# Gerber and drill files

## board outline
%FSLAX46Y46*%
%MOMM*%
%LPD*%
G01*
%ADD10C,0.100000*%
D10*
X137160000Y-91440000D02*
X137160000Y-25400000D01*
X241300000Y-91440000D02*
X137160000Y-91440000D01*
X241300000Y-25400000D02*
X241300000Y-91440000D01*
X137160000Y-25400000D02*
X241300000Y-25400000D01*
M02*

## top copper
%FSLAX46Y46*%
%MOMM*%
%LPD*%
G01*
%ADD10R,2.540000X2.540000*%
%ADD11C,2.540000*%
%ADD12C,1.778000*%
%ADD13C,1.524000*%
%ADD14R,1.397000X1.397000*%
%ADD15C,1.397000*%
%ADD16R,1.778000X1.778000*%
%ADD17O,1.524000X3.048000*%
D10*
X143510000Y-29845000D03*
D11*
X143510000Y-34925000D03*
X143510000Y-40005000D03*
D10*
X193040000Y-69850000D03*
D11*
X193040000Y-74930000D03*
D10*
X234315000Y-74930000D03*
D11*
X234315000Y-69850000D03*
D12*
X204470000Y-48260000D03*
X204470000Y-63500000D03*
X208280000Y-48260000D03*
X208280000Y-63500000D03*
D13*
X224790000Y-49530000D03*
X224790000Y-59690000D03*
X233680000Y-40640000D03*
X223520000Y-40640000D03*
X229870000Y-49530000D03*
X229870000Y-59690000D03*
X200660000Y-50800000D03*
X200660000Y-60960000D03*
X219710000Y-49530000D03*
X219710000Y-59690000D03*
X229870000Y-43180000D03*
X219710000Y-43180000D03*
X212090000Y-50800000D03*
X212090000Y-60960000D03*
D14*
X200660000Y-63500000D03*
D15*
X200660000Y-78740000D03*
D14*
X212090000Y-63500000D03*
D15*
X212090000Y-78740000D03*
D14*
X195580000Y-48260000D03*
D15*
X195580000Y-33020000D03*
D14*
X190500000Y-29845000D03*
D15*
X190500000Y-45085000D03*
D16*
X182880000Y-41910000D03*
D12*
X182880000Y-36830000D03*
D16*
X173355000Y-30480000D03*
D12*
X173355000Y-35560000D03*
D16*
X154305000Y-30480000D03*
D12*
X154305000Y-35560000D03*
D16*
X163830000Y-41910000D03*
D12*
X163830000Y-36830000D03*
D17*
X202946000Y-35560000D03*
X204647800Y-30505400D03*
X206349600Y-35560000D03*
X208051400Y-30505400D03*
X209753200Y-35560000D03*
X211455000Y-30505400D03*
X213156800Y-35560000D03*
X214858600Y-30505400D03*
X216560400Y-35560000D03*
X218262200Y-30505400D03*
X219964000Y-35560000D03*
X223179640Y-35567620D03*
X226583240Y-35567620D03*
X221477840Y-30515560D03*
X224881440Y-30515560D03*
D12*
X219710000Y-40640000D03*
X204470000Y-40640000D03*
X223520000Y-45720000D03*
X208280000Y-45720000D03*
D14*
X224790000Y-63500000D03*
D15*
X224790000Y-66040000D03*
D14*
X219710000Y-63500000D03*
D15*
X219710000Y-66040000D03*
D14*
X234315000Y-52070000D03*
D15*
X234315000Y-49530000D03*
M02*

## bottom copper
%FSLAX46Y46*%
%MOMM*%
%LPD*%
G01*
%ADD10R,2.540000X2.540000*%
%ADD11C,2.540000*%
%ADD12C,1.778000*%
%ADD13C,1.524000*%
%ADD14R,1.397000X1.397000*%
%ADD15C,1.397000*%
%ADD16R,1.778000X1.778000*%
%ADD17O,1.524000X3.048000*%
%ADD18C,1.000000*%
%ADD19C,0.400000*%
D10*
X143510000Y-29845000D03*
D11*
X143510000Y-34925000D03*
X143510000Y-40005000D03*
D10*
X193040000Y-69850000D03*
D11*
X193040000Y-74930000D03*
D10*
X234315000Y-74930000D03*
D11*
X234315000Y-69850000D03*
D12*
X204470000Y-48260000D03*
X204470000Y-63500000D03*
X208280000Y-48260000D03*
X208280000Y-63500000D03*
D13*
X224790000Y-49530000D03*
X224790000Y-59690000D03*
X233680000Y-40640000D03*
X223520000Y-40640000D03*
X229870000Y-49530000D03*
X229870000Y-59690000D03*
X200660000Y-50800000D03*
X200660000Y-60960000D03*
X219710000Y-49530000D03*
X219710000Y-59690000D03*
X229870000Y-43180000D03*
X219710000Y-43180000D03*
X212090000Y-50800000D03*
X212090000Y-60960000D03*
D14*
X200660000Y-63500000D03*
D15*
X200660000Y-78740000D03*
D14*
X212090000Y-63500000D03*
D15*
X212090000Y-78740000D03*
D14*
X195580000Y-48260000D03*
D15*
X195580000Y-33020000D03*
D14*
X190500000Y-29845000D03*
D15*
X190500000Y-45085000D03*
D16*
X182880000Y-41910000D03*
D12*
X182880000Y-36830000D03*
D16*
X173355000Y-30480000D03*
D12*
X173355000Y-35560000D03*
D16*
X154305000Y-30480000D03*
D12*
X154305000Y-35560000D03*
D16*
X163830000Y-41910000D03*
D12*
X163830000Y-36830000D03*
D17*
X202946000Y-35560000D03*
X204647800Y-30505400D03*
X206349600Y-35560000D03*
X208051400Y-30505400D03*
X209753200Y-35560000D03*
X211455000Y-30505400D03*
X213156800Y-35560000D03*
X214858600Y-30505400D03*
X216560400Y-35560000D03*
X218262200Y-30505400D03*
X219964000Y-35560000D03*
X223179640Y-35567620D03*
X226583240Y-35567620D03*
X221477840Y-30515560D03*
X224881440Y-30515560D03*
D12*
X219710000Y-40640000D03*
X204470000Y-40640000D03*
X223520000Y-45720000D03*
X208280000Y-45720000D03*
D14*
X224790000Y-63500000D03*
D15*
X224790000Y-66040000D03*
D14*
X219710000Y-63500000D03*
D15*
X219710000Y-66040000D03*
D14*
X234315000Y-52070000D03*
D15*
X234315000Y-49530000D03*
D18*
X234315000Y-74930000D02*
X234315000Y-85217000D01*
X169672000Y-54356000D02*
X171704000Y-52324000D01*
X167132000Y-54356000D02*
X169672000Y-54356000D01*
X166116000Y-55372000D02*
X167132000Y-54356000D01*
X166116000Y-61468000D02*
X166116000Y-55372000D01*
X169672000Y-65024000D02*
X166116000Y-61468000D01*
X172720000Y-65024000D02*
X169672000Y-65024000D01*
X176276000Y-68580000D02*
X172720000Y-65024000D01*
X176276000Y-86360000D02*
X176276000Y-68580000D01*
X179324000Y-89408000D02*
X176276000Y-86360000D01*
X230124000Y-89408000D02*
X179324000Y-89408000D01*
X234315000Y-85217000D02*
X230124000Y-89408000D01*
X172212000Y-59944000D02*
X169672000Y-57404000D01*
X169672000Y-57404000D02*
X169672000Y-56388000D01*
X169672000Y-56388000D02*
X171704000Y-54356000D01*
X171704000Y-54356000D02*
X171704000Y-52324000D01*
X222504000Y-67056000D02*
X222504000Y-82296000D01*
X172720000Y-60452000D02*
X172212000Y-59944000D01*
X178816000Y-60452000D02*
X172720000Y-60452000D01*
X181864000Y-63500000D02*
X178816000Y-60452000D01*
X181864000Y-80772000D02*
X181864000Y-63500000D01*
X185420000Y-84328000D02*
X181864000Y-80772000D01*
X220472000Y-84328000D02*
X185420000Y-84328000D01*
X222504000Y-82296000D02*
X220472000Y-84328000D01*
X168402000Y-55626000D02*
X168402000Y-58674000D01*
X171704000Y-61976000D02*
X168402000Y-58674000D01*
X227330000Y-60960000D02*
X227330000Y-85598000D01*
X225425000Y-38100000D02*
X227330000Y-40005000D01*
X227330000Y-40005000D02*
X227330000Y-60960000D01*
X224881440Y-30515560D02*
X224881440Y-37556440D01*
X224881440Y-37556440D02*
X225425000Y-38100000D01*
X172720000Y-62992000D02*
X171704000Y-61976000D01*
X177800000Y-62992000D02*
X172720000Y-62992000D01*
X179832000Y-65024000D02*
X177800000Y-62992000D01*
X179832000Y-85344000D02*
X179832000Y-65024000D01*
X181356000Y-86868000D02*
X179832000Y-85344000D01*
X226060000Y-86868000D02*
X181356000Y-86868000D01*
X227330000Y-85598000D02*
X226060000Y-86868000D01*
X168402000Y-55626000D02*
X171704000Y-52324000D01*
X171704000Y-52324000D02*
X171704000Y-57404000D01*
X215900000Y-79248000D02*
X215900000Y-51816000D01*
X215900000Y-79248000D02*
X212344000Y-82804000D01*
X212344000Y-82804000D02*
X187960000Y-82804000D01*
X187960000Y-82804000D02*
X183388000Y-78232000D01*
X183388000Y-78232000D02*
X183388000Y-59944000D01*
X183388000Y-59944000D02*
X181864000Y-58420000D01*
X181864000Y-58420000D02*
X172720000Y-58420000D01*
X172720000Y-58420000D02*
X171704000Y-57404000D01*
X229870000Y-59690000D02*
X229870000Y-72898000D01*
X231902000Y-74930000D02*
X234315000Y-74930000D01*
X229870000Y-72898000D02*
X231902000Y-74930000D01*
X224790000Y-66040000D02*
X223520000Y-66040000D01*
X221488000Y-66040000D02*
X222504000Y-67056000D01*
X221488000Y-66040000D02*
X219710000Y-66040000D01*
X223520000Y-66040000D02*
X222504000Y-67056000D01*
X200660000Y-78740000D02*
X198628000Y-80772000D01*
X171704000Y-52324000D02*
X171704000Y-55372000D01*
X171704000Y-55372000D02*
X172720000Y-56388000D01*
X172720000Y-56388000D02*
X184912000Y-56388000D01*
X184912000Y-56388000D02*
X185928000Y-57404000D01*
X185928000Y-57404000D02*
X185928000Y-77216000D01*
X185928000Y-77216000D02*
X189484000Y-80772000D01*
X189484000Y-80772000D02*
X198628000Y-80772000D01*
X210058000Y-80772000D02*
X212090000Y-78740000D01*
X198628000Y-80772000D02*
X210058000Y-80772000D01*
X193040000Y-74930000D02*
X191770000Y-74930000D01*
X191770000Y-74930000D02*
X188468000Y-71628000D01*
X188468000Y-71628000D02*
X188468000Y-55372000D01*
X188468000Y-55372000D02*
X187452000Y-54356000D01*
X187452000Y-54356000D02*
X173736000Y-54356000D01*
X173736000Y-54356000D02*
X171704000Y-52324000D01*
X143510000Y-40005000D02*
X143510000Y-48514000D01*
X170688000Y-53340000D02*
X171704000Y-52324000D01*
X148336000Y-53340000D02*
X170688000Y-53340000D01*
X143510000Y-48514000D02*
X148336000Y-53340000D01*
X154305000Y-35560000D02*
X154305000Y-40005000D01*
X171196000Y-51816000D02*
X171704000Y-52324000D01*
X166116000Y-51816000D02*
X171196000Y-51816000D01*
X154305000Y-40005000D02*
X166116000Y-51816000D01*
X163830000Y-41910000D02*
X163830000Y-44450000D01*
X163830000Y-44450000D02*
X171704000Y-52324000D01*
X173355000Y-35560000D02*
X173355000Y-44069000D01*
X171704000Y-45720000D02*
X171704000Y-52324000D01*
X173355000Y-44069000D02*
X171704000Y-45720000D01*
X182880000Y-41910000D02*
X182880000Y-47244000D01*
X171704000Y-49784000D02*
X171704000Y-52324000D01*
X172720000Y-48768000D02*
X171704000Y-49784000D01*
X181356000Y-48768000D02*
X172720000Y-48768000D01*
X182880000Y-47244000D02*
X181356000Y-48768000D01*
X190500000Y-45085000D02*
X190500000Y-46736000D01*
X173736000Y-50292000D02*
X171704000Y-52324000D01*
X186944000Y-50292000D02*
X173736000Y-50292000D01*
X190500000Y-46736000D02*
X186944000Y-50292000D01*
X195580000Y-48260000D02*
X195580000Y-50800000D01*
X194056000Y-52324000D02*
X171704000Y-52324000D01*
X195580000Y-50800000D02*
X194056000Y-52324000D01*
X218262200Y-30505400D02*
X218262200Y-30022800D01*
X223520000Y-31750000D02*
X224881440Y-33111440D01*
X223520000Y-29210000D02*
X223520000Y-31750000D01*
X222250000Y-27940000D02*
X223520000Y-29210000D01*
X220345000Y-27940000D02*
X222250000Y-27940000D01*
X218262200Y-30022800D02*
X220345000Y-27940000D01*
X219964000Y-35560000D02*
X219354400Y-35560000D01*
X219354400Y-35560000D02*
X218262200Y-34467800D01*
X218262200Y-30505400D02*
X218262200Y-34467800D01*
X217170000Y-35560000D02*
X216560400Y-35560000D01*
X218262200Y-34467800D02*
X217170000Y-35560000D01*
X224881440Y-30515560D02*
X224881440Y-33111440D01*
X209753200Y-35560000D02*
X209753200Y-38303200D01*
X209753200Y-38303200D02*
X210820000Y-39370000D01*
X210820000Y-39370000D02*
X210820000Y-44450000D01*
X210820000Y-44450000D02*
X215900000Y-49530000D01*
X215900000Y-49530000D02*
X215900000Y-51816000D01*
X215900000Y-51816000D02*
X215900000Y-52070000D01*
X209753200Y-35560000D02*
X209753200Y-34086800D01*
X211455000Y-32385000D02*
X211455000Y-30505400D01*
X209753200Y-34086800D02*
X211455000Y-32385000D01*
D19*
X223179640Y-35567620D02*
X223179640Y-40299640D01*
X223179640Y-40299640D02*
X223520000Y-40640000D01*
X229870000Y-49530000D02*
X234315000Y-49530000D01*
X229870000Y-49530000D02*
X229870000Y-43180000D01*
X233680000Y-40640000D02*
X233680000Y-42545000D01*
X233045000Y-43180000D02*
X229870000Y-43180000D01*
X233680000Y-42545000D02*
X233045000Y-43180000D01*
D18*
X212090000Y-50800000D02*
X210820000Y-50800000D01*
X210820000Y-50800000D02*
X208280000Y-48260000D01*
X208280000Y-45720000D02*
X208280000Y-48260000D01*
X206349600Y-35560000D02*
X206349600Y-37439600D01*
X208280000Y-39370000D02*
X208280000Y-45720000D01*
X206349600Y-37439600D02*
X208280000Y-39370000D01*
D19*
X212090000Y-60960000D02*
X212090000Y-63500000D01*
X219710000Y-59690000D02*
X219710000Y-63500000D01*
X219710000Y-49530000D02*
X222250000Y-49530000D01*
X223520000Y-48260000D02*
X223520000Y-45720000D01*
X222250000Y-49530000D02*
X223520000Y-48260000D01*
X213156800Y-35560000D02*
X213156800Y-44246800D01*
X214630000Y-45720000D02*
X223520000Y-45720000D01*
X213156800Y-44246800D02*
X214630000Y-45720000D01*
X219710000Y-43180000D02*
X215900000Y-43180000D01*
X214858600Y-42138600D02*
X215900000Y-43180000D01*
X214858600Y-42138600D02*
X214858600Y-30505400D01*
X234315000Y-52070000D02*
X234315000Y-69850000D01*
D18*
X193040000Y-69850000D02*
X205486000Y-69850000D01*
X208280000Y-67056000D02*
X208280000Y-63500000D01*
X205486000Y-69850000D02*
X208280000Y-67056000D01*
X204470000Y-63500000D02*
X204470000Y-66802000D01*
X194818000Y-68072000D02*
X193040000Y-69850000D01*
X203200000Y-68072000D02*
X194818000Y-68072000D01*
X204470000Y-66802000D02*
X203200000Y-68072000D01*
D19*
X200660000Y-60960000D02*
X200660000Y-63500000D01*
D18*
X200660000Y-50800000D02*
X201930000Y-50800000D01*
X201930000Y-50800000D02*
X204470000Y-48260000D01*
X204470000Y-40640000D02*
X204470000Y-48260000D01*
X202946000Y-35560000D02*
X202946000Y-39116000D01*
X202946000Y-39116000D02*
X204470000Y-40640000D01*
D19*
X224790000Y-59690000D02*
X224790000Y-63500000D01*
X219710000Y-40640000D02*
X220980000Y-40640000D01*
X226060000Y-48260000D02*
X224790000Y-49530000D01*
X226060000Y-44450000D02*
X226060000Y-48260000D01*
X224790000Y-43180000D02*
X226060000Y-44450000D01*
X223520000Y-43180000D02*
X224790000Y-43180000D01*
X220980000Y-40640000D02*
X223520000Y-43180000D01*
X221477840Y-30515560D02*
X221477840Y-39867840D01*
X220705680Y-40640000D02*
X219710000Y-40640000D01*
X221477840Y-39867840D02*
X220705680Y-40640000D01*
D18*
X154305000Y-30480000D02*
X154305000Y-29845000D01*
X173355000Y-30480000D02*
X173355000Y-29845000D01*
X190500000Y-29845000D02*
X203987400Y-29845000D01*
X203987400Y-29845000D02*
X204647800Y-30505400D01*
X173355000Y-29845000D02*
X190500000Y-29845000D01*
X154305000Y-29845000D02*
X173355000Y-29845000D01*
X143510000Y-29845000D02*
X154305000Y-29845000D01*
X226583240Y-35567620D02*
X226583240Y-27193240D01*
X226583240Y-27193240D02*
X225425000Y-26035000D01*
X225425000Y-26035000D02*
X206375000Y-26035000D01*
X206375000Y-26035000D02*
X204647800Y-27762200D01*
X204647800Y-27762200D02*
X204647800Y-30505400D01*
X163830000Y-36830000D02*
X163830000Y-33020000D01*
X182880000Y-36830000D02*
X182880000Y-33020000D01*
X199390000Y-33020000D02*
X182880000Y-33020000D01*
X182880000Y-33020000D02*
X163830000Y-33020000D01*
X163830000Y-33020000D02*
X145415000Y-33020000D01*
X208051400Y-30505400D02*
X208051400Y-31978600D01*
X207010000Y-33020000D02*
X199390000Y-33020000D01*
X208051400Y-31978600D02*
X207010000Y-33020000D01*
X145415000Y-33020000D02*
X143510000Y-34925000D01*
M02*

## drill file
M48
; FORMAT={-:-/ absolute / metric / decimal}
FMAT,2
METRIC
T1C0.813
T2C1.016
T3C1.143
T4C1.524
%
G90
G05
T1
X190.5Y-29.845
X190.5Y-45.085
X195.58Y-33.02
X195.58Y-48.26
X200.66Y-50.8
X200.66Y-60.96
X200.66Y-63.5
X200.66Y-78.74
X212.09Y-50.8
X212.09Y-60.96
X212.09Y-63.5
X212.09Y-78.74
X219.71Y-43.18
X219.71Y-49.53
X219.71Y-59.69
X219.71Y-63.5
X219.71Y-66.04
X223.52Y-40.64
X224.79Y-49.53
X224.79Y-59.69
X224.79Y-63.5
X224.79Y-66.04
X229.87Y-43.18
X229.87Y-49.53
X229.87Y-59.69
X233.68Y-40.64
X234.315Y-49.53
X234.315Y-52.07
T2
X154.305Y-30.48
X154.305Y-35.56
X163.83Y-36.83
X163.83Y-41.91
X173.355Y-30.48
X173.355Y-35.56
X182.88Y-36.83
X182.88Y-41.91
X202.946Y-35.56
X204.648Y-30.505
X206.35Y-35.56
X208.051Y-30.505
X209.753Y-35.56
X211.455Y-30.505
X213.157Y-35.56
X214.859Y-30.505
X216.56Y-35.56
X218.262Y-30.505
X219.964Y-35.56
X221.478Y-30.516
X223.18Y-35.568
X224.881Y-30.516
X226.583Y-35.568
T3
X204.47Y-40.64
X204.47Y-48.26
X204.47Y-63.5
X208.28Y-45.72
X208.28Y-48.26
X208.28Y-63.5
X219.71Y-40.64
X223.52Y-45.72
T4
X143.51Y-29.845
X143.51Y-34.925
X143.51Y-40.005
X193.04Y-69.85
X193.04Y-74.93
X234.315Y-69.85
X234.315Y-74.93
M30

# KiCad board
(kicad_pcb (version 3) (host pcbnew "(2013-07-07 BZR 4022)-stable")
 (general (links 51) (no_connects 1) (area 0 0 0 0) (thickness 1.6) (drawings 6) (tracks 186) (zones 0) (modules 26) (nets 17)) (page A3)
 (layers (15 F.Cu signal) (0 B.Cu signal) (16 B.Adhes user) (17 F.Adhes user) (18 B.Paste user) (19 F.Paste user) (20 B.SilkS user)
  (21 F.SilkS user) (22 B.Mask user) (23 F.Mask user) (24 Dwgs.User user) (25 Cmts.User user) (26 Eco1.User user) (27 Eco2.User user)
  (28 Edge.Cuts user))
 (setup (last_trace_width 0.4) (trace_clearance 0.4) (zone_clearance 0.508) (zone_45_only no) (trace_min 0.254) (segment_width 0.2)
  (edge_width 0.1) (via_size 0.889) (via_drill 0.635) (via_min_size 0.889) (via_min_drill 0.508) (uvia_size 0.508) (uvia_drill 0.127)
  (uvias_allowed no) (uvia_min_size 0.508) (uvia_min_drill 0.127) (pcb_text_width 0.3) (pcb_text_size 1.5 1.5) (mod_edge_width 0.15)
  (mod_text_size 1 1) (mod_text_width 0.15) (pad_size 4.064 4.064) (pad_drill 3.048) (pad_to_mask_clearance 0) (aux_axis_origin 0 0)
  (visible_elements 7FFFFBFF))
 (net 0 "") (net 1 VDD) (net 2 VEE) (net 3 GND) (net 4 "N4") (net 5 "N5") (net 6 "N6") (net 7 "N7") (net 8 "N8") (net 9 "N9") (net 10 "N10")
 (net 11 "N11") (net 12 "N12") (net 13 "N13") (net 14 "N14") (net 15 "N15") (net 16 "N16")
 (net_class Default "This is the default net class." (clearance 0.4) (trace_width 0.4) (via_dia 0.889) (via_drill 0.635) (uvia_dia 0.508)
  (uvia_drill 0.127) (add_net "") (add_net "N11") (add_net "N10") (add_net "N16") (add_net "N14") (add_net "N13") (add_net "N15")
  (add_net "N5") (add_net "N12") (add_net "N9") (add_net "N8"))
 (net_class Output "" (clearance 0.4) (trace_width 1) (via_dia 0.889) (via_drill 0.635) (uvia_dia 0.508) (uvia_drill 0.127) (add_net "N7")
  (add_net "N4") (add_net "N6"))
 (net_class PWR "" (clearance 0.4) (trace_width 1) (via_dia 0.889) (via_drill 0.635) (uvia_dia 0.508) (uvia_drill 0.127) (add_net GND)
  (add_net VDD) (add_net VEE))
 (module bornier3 (layer F.Cu) (at 143.51 34.925 270)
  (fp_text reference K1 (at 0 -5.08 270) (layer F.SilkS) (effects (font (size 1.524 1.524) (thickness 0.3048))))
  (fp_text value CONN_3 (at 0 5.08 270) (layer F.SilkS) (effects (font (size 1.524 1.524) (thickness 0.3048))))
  (pad 1 thru_hole rect (at -5.08 0 270) (size 2.54 2.54) (drill 1.524) (layers *.Cu *.Mask F.SilkS) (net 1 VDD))
  (pad 2 thru_hole circle (at 0 0 270) (size 2.54 2.54) (drill 1.524) (layers *.Cu *.Mask F.SilkS) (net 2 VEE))
  (pad 3 thru_hole circle (at 5.08 0 270) (size 2.54 2.54) (drill 1.524) (layers *.Cu *.Mask F.SilkS) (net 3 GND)))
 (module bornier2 (layer F.Cu) (at 193.04 72.39 270)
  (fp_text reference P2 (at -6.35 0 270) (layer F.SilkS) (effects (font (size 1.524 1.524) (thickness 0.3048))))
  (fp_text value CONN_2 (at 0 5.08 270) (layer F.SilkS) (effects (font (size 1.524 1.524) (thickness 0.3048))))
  (pad 1 thru_hole rect (at -2.54 0 270) (size 2.54 2.54) (drill 1.524) (layers *.Cu *.Mask F.SilkS) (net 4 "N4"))
  (pad 2 thru_hole circle (at 2.54 0 270) (size 2.54 2.54) (drill 1.524) (layers *.Cu *.Mask F.SilkS) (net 3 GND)))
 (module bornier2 (layer F.Cu) (at 234.315 72.39 90)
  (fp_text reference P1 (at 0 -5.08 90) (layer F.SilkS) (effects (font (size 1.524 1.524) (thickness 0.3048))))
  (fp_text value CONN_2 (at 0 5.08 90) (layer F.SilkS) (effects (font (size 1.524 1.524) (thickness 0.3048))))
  (pad 1 thru_hole rect (at -2.54 0 90) (size 2.54 2.54) (drill 1.524) (layers *.Cu *.Mask F.SilkS) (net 3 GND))
  (pad 2 thru_hole circle (at 2.54 0 90) (size 2.54 2.54) (drill 1.524) (layers *.Cu *.Mask F.SilkS) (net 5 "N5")))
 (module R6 (layer F.Cu) (at 204.47 55.88 270) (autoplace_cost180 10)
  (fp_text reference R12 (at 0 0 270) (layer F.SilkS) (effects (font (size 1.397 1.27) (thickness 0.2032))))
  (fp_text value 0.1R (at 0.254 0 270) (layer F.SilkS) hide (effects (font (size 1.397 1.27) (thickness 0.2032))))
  (pad 1 thru_hole circle (at -7.62 0 270) (size 1.778 1.778) (drill 1.143) (layers *.Cu *.Mask F.SilkS) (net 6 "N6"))
  (pad 2 thru_hole circle (at 7.62 0 270) (size 1.778 1.778) (drill 1.143) (layers *.Cu *.Mask F.SilkS) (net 4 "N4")))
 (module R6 (layer F.Cu) (at 208.28 55.88 270) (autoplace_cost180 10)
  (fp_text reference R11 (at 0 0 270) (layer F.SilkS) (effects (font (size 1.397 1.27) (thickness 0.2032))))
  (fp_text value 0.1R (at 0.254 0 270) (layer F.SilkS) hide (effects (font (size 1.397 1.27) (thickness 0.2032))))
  (pad 1 thru_hole circle (at -7.62 0 270) (size 1.778 1.778) (drill 1.143) (layers *.Cu *.Mask F.SilkS) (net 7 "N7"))
  (pad 2 thru_hole circle (at 7.62 0 270) (size 1.778 1.778) (drill 1.143) (layers *.Cu *.Mask F.SilkS) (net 4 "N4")))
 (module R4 (layer F.Cu) (at 224.79 54.61 270) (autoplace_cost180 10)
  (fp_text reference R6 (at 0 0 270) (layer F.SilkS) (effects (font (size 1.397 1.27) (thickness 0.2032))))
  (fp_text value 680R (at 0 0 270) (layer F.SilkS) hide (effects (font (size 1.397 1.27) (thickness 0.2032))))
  (pad 1 thru_hole circle (at -5.08 0 270) (size 1.524 1.524) (drill 0.8128) (layers *.Cu *.Mask F.SilkS) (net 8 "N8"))
  (pad 2 thru_hole circle (at 5.08 0 270) (size 1.524 1.524) (drill 0.8128) (layers *.Cu *.Mask F.SilkS) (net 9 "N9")))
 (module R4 (layer F.Cu) (at 228.6 40.64 180) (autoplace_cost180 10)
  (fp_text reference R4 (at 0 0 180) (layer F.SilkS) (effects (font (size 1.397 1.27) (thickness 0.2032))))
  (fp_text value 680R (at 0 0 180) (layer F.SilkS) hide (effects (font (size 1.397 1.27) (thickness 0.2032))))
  (pad 1 thru_hole circle (at -5.08 0 180) (size 1.524 1.524) (drill 0.8128) (layers *.Cu *.Mask F.SilkS) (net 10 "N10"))
  (pad 2 thru_hole circle (at 5.08 0 180) (size 1.524 1.524) (drill 0.8128) (layers *.Cu *.Mask F.SilkS) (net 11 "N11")))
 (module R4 (layer F.Cu) (at 229.87 54.61 270) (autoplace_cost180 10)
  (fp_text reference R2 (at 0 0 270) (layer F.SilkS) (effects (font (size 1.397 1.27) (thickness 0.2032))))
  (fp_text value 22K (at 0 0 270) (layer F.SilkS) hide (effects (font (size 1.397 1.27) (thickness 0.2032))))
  (pad 1 thru_hole circle (at -5.08 0 270) (size 1.524 1.524) (drill 0.8128) (layers *.Cu *.Mask F.SilkS) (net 10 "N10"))
  (pad 2 thru_hole circle (at 5.08 0 270) (size 1.524 1.524) (drill 0.8128) (layers *.Cu *.Mask F.SilkS) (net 3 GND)))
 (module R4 (layer F.Cu) (at 200.66 55.88 270) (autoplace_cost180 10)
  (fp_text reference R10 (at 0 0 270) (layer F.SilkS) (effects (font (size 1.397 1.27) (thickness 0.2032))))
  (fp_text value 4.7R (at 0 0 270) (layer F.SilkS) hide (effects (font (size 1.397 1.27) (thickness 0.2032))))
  (pad 1 thru_hole circle (at -5.08 0 270) (size 1.524 1.524) (drill 0.8128) (layers *.Cu *.Mask F.SilkS) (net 6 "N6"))
  (pad 2 thru_hole circle (at 5.08 0 270) (size 1.524 1.524) (drill 0.8128) (layers *.Cu *.Mask F.SilkS) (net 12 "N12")))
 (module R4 (layer F.Cu) (at 219.71 54.61 270) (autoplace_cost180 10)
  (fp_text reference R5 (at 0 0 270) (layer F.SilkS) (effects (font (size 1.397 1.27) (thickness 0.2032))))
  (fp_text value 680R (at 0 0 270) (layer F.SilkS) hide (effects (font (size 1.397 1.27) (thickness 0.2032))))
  (pad 1 thru_hole circle (at -5.08 0 270) (size 1.524 1.524) (drill 0.8128) (layers *.Cu *.Mask F.SilkS) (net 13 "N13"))
  (pad 2 thru_hole circle (at 5.08 0 270) (size 1.524 1.524) (drill 0.8128) (layers *.Cu *.Mask F.SilkS) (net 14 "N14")))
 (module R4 (layer F.Cu) (at 224.79 43.18 180) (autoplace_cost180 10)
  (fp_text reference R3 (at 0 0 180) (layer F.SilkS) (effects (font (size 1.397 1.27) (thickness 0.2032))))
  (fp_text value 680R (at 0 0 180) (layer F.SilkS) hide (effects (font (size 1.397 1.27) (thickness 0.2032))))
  (pad 1 thru_hole circle (at -5.08 0 180) (size 1.524 1.524) (drill 0.8128) (layers *.Cu *.Mask F.SilkS) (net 10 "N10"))
  (pad 2 thru_hole circle (at 5.08 0 180) (size 1.524 1.524) (drill 0.8128) (layers *.Cu *.Mask F.SilkS) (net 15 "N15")))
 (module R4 (layer F.Cu) (at 212.09 55.88 270) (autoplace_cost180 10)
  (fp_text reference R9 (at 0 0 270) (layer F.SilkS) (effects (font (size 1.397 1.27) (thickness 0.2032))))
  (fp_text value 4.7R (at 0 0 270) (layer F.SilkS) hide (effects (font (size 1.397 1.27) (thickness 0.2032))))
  (pad 1 thru_hole circle (at -5.08 0 270) (size 1.524 1.524) (drill 0.8128) (layers *.Cu *.Mask F.SilkS) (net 7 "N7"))
  (pad 2 thru_hole circle (at 5.08 0 270) (size 1.524 1.524) (drill 0.8128) (layers *.Cu *.Mask F.SilkS) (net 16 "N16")))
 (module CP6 (layer F.Cu) (at 200.66 71.12 270)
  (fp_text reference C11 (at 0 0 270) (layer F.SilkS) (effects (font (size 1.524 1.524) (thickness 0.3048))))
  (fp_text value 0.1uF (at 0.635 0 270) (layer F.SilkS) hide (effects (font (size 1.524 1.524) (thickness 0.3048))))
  (pad 1 thru_hole rect (at -7.62 0 270) (size 1.397 1.397) (drill 0.8128) (layers *.Cu *.Mask F.SilkS) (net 12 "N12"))
  (pad 2 thru_hole circle (at 7.62 0 270) (size 1.397 1.397) (drill 0.8128) (layers *.Cu *.Mask F.SilkS) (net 3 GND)))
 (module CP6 (layer F.Cu) (at 212.09 71.12 270)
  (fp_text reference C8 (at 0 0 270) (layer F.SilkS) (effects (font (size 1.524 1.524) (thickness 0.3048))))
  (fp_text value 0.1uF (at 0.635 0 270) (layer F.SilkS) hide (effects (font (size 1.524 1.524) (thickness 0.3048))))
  (pad 1 thru_hole rect (at -7.62 0 270) (size 1.397 1.397) (drill 0.8128) (layers *.Cu *.Mask F.SilkS) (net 16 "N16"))
  (pad 2 thru_hole circle (at 7.62 0 270) (size 1.397 1.397) (drill 0.8128) (layers *.Cu *.Mask F.SilkS) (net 3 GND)))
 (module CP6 (layer F.Cu) (at 195.58 40.64 90)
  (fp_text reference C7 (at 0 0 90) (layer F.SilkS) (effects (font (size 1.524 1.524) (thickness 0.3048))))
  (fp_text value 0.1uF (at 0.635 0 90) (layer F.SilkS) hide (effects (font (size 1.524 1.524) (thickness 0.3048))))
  (pad 1 thru_hole rect (at -7.62 0 90) (size 1.397 1.397) (drill 0.8128) (layers *.Cu *.Mask F.SilkS) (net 3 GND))
  (pad 2 thru_hole circle (at 7.62 0 90) (size 1.397 1.397) (drill 0.8128) (layers *.Cu *.Mask F.SilkS) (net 2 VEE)))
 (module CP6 (layer F.Cu) (at 190.5 37.465 270)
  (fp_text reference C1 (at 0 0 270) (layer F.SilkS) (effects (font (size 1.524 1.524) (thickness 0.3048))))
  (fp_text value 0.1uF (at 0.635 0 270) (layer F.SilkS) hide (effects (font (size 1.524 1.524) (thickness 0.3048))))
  (pad 1 thru_hole rect (at -7.62 0 270) (size 1.397 1.397) (drill 0.8128) (layers *.Cu *.Mask F.SilkS) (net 1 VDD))
  (pad 2 thru_hole circle (at 7.62 0 270) (size 1.397 1.397) (drill 0.8128) (layers *.Cu *.Mask F.SilkS) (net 3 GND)))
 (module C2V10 (layer F.Cu) (at 182.88 39.37 90)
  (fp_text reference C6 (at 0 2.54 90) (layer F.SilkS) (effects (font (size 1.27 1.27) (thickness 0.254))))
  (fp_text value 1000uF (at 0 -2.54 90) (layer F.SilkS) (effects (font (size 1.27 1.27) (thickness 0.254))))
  (pad 1 thru_hole rect (at -2.54 0 90) (size 1.778 1.778) (drill 1.016) (layers *.Cu *.Mask F.SilkS) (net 3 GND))
  (pad 2 thru_hole circle (at 2.54 0 90) (size 1.778 1.778) (drill 1.016) (layers *.Cu *.Mask F.SilkS) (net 2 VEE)))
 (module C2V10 (layer F.Cu) (at 173.355 33.02 270)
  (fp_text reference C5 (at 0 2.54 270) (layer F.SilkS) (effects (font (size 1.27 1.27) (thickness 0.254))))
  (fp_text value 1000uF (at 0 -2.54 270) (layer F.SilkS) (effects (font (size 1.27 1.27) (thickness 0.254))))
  (pad 1 thru_hole rect (at -2.54 0 270) (size 1.778 1.778) (drill 1.016) (layers *.Cu *.Mask F.SilkS) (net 1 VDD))
  (pad 2 thru_hole circle (at 2.54 0 270) (size 1.778 1.778) (drill 1.016) (layers *.Cu *.Mask F.SilkS) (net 3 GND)))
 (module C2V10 (layer F.Cu) (at 154.305 33.02 270)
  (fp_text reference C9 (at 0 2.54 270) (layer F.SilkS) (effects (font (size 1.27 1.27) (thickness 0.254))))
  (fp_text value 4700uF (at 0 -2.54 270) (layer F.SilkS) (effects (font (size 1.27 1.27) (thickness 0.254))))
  (pad 1 thru_hole rect (at -2.54 0 270) (size 1.778 1.778) (drill 1.016) (layers *.Cu *.Mask F.SilkS) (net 1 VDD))
  (pad 2 thru_hole circle (at 2.54 0 270) (size 1.778 1.778) (drill 1.016) (layers *.Cu *.Mask F.SilkS) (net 3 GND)))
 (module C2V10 (layer F.Cu) (at 163.83 39.37 90)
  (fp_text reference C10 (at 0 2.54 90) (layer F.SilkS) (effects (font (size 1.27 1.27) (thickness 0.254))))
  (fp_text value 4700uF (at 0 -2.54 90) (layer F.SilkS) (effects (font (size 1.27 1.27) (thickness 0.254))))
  (pad 1 thru_hole rect (at -2.54 0 90) (size 1.778 1.778) (drill 1.016) (layers *.Cu *.Mask F.SilkS) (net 3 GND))
  (pad 2 thru_hole circle (at 2.54 0 90) (size 1.778 1.778) (drill 1.016) (layers *.Cu *.Mask F.SilkS) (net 2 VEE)))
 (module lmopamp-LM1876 (layer F.Cu) (at 213.995 33.655)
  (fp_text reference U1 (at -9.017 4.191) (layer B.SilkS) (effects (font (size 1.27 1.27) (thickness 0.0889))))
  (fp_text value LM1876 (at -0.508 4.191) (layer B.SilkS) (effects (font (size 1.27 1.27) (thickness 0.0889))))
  (pad 1 thru_hole oval (at -11.049 1.905) (size 1.524 3.048) (drill 1.016) (layers *.Cu F.Paste F.SilkS F.Mask) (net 6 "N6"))
  (pad 2 thru_hole oval (at -9.3472 -3.1496) (size 1.524 3.048) (drill 1.016) (layers *.Cu F.Paste F.SilkS F.Mask) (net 1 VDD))
  (pad 3 thru_hole oval (at -7.6454 1.905) (size 1.524 3.048) (drill 1.016) (layers *.Cu F.Paste F.SilkS F.Mask) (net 7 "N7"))
  (pad 4 thru_hole oval (at -5.9436 -3.1496) (size 1.524 3.048) (drill 1.016) (layers *.Cu F.Paste F.SilkS F.Mask) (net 2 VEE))
  (pad 5 thru_hole oval (at -4.2418 1.905) (size 1.524 3.048) (drill 1.016) (layers *.Cu F.Paste F.SilkS F.Mask) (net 3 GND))
  (pad 6 thru_hole oval (at -2.54 -3.1496) (size 1.524 3.048) (drill 1.016) (layers *.Cu F.Paste F.SilkS F.Mask) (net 3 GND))
  (pad 7 thru_hole oval (at -0.8382 1.905) (size 1.524 3.048) (drill 1.016) (layers *.Cu F.Paste F.SilkS F.Mask) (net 13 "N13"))
  (pad 8 thru_hole oval (at 0.8636 -3.1496) (size 1.524 3.048) (drill 1.016) (layers *.Cu F.Paste F.SilkS F.Mask) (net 15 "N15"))
  (pad 9 thru_hole oval (at 2.5654 1.905) (size 1.524 3.048) (drill 1.016) (layers *.Cu F.Paste F.SilkS F.Mask) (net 3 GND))
  (pad 10 thru_hole oval (at 4.2672 -3.1496) (size 1.524 3.048) (drill 1.016) (layers *.Cu F.Paste F.SilkS F.Mask) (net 3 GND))
  (pad 11 thru_hole oval (at 5.969 1.905) (size 1.524 3.048) (drill 1.016) (layers *.Cu F.Paste F.SilkS F.Mask) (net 3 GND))
  (pad 13 thru_hole oval (at 9.18464 1.91262) (size 1.524 3.048) (drill 1.016) (layers *.Cu F.Paste F.SilkS F.Mask) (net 11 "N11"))
  (pad 15 thru_hole oval (at 12.58824 1.91262) (size 1.524 3.048) (drill 1.016) (layers *.Cu F.Paste F.SilkS F.Mask) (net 1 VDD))
  (pad 12 thru_hole oval (at 7.48284 -3.13944) (size 1.524 3.048) (drill 1.016) (layers *.Cu F.Paste F.SilkS F.Mask) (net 8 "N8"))
  (pad 14 thru_hole oval (at 10.88644 -3.13944) (size 1.524 3.048) (drill 1.016) (layers *.Cu F.Paste F.SilkS F.Mask) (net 3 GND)))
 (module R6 (layer F.Cu) (at 212.09 40.64 180) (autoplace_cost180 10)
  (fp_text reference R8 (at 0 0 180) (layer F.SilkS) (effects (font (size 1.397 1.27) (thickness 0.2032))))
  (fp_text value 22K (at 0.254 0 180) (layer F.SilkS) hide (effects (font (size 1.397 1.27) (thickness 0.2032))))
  (pad 1 thru_hole circle (at -7.62 0 180) (size 1.778 1.778) (drill 1.143) (layers *.Cu *.Mask F.SilkS) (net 8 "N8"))
  (pad 2 thru_hole circle (at 7.62 0 180) (size 1.778 1.778) (drill 1.143) (layers *.Cu *.Mask F.SilkS) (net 6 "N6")))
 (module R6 (layer F.Cu) (at 215.9 45.72 180) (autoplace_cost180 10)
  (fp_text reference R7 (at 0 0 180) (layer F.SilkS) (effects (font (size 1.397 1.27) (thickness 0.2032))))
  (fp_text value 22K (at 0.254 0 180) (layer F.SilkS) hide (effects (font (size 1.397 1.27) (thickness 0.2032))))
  (pad 1 thru_hole circle (at -7.62 0 180) (size 1.778 1.778) (drill 1.143) (layers *.Cu *.Mask F.SilkS) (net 13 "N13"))
  (pad 2 thru_hole circle (at 7.62 0 180) (size 1.778 1.778) (drill 1.143) (layers *.Cu *.Mask F.SilkS) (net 7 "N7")))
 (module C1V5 (layer F.Cu) (at 224.79 64.77 270)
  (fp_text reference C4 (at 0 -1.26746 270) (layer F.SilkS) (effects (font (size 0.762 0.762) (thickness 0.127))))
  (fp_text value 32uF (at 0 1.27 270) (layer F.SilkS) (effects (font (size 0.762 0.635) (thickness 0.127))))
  (pad 1 thru_hole rect (at -1.27 0 270) (size 1.397 1.397) (drill 0.8128) (layers *.Cu *.Mask F.SilkS) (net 9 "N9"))
  (pad 2 thru_hole circle (at 1.27 0 270) (size 1.397 1.397) (drill 0.8128) (layers *.Cu *.Mask F.SilkS) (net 3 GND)))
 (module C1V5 (layer F.Cu) (at 219.71 64.77 270)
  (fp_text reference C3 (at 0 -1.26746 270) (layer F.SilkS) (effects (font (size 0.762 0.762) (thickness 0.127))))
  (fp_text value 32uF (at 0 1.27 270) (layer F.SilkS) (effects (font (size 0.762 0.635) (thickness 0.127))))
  (pad 1 thru_hole rect (at -1.27 0 270) (size 1.397 1.397) (drill 0.8128) (layers *.Cu *.Mask F.SilkS) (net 14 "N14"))
  (pad 2 thru_hole circle (at 1.27 0 270) (size 1.397 1.397) (drill 0.8128) (layers *.Cu *.Mask F.SilkS) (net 3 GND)))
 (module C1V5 (layer F.Cu) (at 234.315 50.8 90)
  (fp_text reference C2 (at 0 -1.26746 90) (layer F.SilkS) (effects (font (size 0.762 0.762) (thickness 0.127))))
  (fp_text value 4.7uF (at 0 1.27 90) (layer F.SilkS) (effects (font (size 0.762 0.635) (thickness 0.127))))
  (pad 1 thru_hole rect (at -1.27 0 90) (size 1.397 1.397) (drill 0.8128) (layers *.Cu *.Mask F.SilkS) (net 5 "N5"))
  (pad 2 thru_hole circle (at 1.27 0 90) (size 1.397 1.397) (drill 0.8128) (layers *.Cu *.Mask F.SilkS) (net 10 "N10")))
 (gr_line (start 137.16 91.44) (end 137.16 25.4) (angle 90) (layer Edge.Cuts) (width 0.1))
 (gr_line (start 241.3 91.44) (end 137.16 91.44) (angle 90) (layer Edge.Cuts) (width 0.1))
 (gr_line (start 241.3 25.4) (end 241.3 91.44) (angle 90) (layer Edge.Cuts) (width 0.1))
 (gr_line (start 137.16 25.4) (end 241.3 25.4) (angle 90) (layer Edge.Cuts) (width 0.1))
 (segment (start 234.315 74.93) (end 234.315 85.217) (width 1) (layer B.Cu) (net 3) (status 400000))
 (segment (start 169.672 54.356) (end 171.704 52.324) (width 1) (layer B.Cu) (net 3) (status 800000))
 (segment (start 167.132 54.356) (end 169.672 54.356) (width 1) (layer B.Cu) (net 3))
 (segment (start 166.116 55.372) (end 167.132 54.356) (width 1) (layer B.Cu) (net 3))
 (segment (start 166.116 61.468) (end 166.116 55.372) (width 1) (layer B.Cu) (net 3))
 (segment (start 169.672 65.024) (end 166.116 61.468) (width 1) (layer B.Cu) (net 3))
 (segment (start 172.72 65.024) (end 169.672 65.024) (width 1) (layer B.Cu) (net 3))
 (segment (start 176.276 68.58) (end 172.72 65.024) (width 1) (layer B.Cu) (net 3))
 (segment (start 176.276 86.36) (end 176.276 68.58) (width 1) (layer B.Cu) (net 3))
 (segment (start 179.324 89.408) (end 176.276 86.36) (width 1) (layer B.Cu) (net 3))
 (segment (start 230.124 89.408) (end 179.324 89.408) (width 1) (layer B.Cu) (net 3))
 (segment (start 234.315 85.217) (end 230.124 89.408) (width 1) (layer B.Cu) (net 3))
 (segment (start 172.212 59.944) (end 169.672 57.404) (width 1) (layer B.Cu) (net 3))
 (segment (start 169.672 57.404) (end 169.672 56.388) (width 1) (layer B.Cu) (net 3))
 (segment (start 169.672 56.388) (end 171.704 54.356) (width 1) (layer B.Cu) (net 3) (status 800000))
 (segment (start 171.704 54.356) (end 171.704 52.324) (width 1) (layer B.Cu) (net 3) (status C00000))
 (segment (start 222.504 67.056) (end 222.504 82.296) (width 1) (layer B.Cu) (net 3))
 (segment (start 172.72 60.452) (end 172.212 59.944) (width 1) (layer B.Cu) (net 3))
 (segment (start 178.816 60.452) (end 172.72 60.452) (width 1) (layer B.Cu) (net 3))
 (segment (start 181.864 63.5) (end 178.816 60.452) (width 1) (layer B.Cu) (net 3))
 (segment (start 181.864 80.772) (end 181.864 63.5) (width 1) (layer B.Cu) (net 3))
 (segment (start 185.42 84.328) (end 181.864 80.772) (width 1) (layer B.Cu) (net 3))
 (segment (start 220.472 84.328) (end 185.42 84.328) (width 1) (layer B.Cu) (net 3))
 (segment (start 222.504 82.296) (end 220.472 84.328) (width 1) (layer B.Cu) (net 3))
 (segment (start 168.402 55.626) (end 168.402 58.674) (width 1) (layer B.Cu) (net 3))
 (segment (start 171.704 61.976) (end 168.402 58.674) (width 1) (layer B.Cu) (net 3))
 (segment (start 227.33 60.96) (end 227.33 85.598) (width 1) (layer B.Cu) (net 3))
 (segment (start 225.425 38.1) (end 227.33 40.005) (width 1) (layer B.Cu) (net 3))
 (segment (start 227.33 40.005) (end 227.33 60.96) (width 1) (layer B.Cu) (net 3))
 (segment (start 224.88144 30.51556) (end 224.88144 37.55644) (width 1) (layer B.Cu) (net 3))
 (segment (start 224.88144 37.55644) (end 225.425 38.1) (width 1) (layer B.Cu) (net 3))
 (segment (start 172.72 62.992) (end 171.704 61.976) (width 1) (layer B.Cu) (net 3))
 (segment (start 177.8 62.992) (end 172.72 62.992) (width 1) (layer B.Cu) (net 3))
 (segment (start 179.832 65.024) (end 177.8 62.992) (width 1) (layer B.Cu) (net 3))
 (segment (start 179.832 85.344) (end 179.832 65.024) (width 1) (layer B.Cu) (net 3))
 (segment (start 181.356 86.868) (end 179.832 85.344) (width 1) (layer B.Cu) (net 3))
 (segment (start 226.06 86.868) (end 181.356 86.868) (width 1) (layer B.Cu) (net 3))
 (segment (start 227.33 85.598) (end 226.06 86.868) (width 1) (layer B.Cu) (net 3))
 (segment (start 168.402 55.626) (end 171.704 52.324) (width 1) (layer B.Cu) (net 3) (status 800000))
 (segment (start 171.704 52.324) (end 171.704 57.404) (width 1) (layer B.Cu) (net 3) (status 400000))
 (segment (start 215.9 79.248) (end 215.9 51.816) (width 1) (layer B.Cu) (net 3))
 (segment (start 215.9 79.248) (end 212.344 82.804) (width 1) (layer B.Cu) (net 3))
 (segment (start 212.344 82.804) (end 187.96 82.804) (width 1) (layer B.Cu) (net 3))
 (segment (start 187.96 82.804) (end 183.388 78.232) (width 1) (layer B.Cu) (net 3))
 (segment (start 183.388 78.232) (end 183.388 59.944) (width 1) (layer B.Cu) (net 3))
 (segment (start 183.388 59.944) (end 181.864 58.42) (width 1) (layer B.Cu) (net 3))
 (segment (start 181.864 58.42) (end 172.72 58.42) (width 1) (layer B.Cu) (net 3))
 (segment (start 172.72 58.42) (end 171.704 57.404) (width 1) (layer B.Cu) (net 3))
 (segment (start 229.87 59.69) (end 229.87 72.898) (width 1) (layer B.Cu) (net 3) (status 400000))
 (segment (start 231.902 74.93) (end 234.315 74.93) (width 1) (layer B.Cu) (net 3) (status 800000))
 (segment (start 229.87 72.898) (end 231.902 74.93) (width 1) (layer B.Cu) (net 3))
 (segment (start 224.79 66.04) (end 223.52 66.04) (width 1) (layer B.Cu) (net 3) (status 400000))
 (segment (start 221.488 66.04) (end 222.504 67.056) (width 1) (layer B.Cu) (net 3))
 (segment (start 221.488 66.04) (end 219.71 66.04) (width 1) (layer B.Cu) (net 3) (status 800000))
 (segment (start 223.52 66.04) (end 222.504 67.056) (width 1) (layer B.Cu) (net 3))
 (segment (start 200.66 78.74) (end 198.628 80.772) (width 1) (layer B.Cu) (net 3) (status 400000))
 (segment (start 171.704 52.324) (end 171.704 55.372) (width 1) (layer B.Cu) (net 3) (status 400000))
 (segment (start 171.704 55.372) (end 172.72 56.388) (width 1) (layer B.Cu) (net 3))
 (segment (start 172.72 56.388) (end 184.912 56.388) (width 1) (layer B.Cu) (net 3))
 (segment (start 184.912 56.388) (end 185.928 57.404) (width 1) (layer B.Cu) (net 3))
 (segment (start 185.928 57.404) (end 185.928 77.216) (width 1) (layer B.Cu) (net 3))
 (segment (start 185.928 77.216) (end 189.484 80.772) (width 1) (layer B.Cu) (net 3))
 (segment (start 189.484 80.772) (end 198.628 80.772) (width 1) (layer B.Cu) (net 3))
 (segment (start 210.058 80.772) (end 212.09 78.74) (width 1) (layer B.Cu) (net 3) (status 800000))
 (segment (start 198.628 80.772) (end 210.058 80.772) (width 1) (layer B.Cu) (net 3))
 (segment (start 193.04 74.93) (end 191.77 74.93) (width 1) (layer B.Cu) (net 3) (status C00000))
 (segment (start 191.77 74.93) (end 188.468 71.628) (width 1) (layer B.Cu) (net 3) (status 400000))
 (segment (start 188.468 71.628) (end 188.468 55.372) (width 1) (layer B.Cu) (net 3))
 (segment (start 188.468 55.372) (end 187.452 54.356) (width 1) (layer B.Cu) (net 3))
 (segment (start 187.452 54.356) (end 173.736 54.356) (width 1) (layer B.Cu) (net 3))
 (segment (start 173.736 54.356) (end 171.704 52.324) (width 1) (layer B.Cu) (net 3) (status 800000))
 (segment (start 143.51 40.005) (end 143.51 48.514) (width 1) (layer B.Cu) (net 3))
 (segment (start 170.688 53.34) (end 171.704 52.324) (width 1) (layer B.Cu) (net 3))
 (segment (start 148.336 53.34) (end 170.688 53.34) (width 1) (layer B.Cu) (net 3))
 (segment (start 143.51 48.514) (end 148.336 53.34) (width 1) (layer B.Cu) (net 3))
 (segment (start 154.305 35.56) (end 154.305 40.005) (width 1) (layer B.Cu) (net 3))
 (segment (start 171.196 51.816) (end 171.704 52.324) (width 1) (layer B.Cu) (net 3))
 (segment (start 166.116 51.816) (end 171.196 51.816) (width 1) (layer B.Cu) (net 3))
 (segment (start 154.305 40.005) (end 166.116 51.816) (width 1) (layer B.Cu) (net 3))
 (segment (start 163.83 41.91) (end 163.83 44.45) (width 1) (layer B.Cu) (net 3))
 (segment (start 163.83 44.45) (end 171.704 52.324) (width 1) (layer B.Cu) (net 3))
 (segment (start 173.355 35.56) (end 173.355 44.069) (width 1) (layer B.Cu) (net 3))
 (segment (start 171.704 45.72) (end 171.704 52.324) (width 1) (layer B.Cu) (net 3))
 (segment (start 173.355 44.069) (end 171.704 45.72) (width 1) (layer B.Cu) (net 3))
 (segment (start 182.88 41.91) (end 182.88 47.244) (width 1) (layer B.Cu) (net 3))
 (segment (start 171.704 49.784) (end 171.704 52.324) (width 1) (layer B.Cu) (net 3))
 (segment (start 172.72 48.768) (end 171.704 49.784) (width 1) (layer B.Cu) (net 3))
 (segment (start 181.356 48.768) (end 172.72 48.768) (width 1) (layer B.Cu) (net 3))
 (segment (start 182.88 47.244) (end 181.356 48.768) (width 1) (layer B.Cu) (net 3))
 (segment (start 190.5 45.085) (end 190.5 46.736) (width 1) (layer B.Cu) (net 3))
 (segment (start 173.736 50.292) (end 171.704 52.324) (width 1) (layer B.Cu) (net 3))
 (segment (start 186.944 50.292) (end 173.736 50.292) (width 1) (layer B.Cu) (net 3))
 (segment (start 190.5 46.736) (end 186.944 50.292) (width 1) (layer B.Cu) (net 3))
 (segment (start 195.58 48.26) (end 195.58 50.8) (width 1) (layer B.Cu) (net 3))
 (segment (start 194.056 52.324) (end 171.704 52.324) (width 1) (layer B.Cu) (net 3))
 (segment (start 195.58 50.8) (end 194.056 52.324) (width 1) (layer B.Cu) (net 3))
 (segment (start 218.2622 30.5054) (end 218.2622 30.0228) (width 1) (layer B.Cu) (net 3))
 (segment (start 223.52 31.75) (end 224.88144 33.11144) (width 1) (layer B.Cu) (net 3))
 (segment (start 223.52 29.21) (end 223.52 31.75) (width 1) (layer B.Cu) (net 3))
 (segment (start 222.25 27.94) (end 223.52 29.21) (width 1) (layer B.Cu) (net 3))
 (segment (start 220.345 27.94) (end 222.25 27.94) (width 1) (layer B.Cu) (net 3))
 (segment (start 218.2622 30.0228) (end 220.345 27.94) (width 1) (layer B.Cu) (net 3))
 (segment (start 219.964 35.56) (end 219.3544 35.56) (width 1) (layer B.Cu) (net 3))
 (segment (start 219.3544 35.56) (end 218.2622 34.4678) (width 1) (layer B.Cu) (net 3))
 (segment (start 218.2622 30.5054) (end 218.2622 34.4678) (width 1) (layer B.Cu) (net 3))
 (segment (start 217.17 35.56) (end 216.5604 35.56) (width 1) (layer B.Cu) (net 3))
 (segment (start 218.2622 34.4678) (end 217.17 35.56) (width 1) (layer B.Cu) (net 3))
 (segment (start 224.88144 30.51556) (end 224.88144 33.11144) (width 1) (layer B.Cu) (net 3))
 (segment (start 209.7532 35.56) (end 209.7532 38.3032) (width 1) (layer B.Cu) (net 3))
 (segment (start 209.7532 38.3032) (end 210.82 39.37) (width 1) (layer B.Cu) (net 3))
 (segment (start 210.82 39.37) (end 210.82 44.45) (width 1) (layer B.Cu) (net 3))
 (segment (start 210.82 44.45) (end 215.9 49.53) (width 1) (layer B.Cu) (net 3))
 (segment (start 215.9 49.53) (end 215.9 51.816) (width 1) (layer B.Cu) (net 3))
 (segment (start 215.9 51.816) (end 215.9 52.07) (width 1) (layer B.Cu) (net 3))
 (segment (start 209.7532 35.56) (end 209.7532 34.0868) (width 1) (layer B.Cu) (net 3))
 (segment (start 211.455 32.385) (end 211.455 30.5054) (width 1) (layer B.Cu) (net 3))
 (segment (start 209.7532 34.0868) (end 211.455 32.385) (width 1) (layer B.Cu) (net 3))
 (segment (start 223.17964 35.56762) (end 223.17964 40.29964) (width 0.4) (layer B.Cu) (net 11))
 (segment (start 223.17964 40.29964) (end 223.52 40.64) (width 0.4) (layer B.Cu) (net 11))
 (segment (start 229.87 49.53) (end 234.315 49.53) (width 0.4) (layer B.Cu) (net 10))
 (segment (start 229.87 49.53) (end 229.87 43.18) (width 0.4) (layer B.Cu) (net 10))
 (segment (start 233.68 40.64) (end 233.68 42.545) (width 0.4) (layer B.Cu) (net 10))
 (segment (start 233.045 43.18) (end 229.87 43.18) (width 0.4) (layer B.Cu) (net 10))
 (segment (start 233.68 42.545) (end 233.045 43.18) (width 0.4) (layer B.Cu) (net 10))
 (segment (start 212.09 50.8) (end 210.82 50.8) (width 1) (layer B.Cu) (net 7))
 (segment (start 210.82 50.8) (end 208.28 48.26) (width 1) (layer B.Cu) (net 7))
 (segment (start 208.28 45.72) (end 208.28 48.26) (width 1) (layer B.Cu) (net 7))
 (segment (start 206.3496 35.56) (end 206.3496 37.4396) (width 1) (layer B.Cu) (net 7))
 (segment (start 208.28 39.37) (end 208.28 45.72) (width 1) (layer B.Cu) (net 7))
 (segment (start 206.3496 37.4396) (end 208.28 39.37) (width 1) (layer B.Cu) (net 7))
 (segment (start 212.09 60.96) (end 212.09 63.5) (width 0.4) (layer B.Cu) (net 16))
 (segment (start 219.71 59.69) (end 219.71 63.5) (width 0.4) (layer B.Cu) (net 14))
 (segment (start 219.71 49.53) (end 222.25 49.53) (width 0.4) (layer B.Cu) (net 13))
 (segment (start 223.52 48.26) (end 223.52 45.72) (width 0.4) (layer B.Cu) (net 13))
 (segment (start 222.25 49.53) (end 223.52 48.26) (width 0.4) (layer B.Cu) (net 13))
 (segment (start 213.1568 35.56) (end 213.1568 44.2468) (width 0.4) (layer B.Cu) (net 13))
 (segment (start 214.63 45.72) (end 223.52 45.72) (width 0.4) (layer B.Cu) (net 13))
 (segment (start 213.1568 44.2468) (end 214.63 45.72) (width 0.4) (layer B.Cu) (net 13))
 (segment (start 219.71 43.18) (end 215.9 43.18) (width 0.4) (layer B.Cu) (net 15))
 (segment (start 214.8586 42.1386) (end 215.9 43.18) (width 0.4) (layer B.Cu) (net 15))
 (segment (start 214.8586 42.1386) (end 214.8586 30.5054) (width 0.4) (layer B.Cu) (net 15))
 (segment (start 234.315 52.07) (end 234.315 69.85) (width 0.4) (layer B.Cu) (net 5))
 (segment (start 193.04 69.85) (end 205.486 69.85) (width 1) (layer B.Cu) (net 4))
 (segment (start 208.28 67.056) (end 208.28 63.5) (width 1) (layer B.Cu) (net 4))
 (segment (start 205.486 69.85) (end 208.28 67.056) (width 1) (layer B.Cu) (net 4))
 (segment (start 204.47 63.5) (end 204.47 66.802) (width 1) (layer B.Cu) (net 4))
 (segment (start 194.818 68.072) (end 193.04 69.85) (width 1) (layer B.Cu) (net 4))
 (segment (start 203.2 68.072) (end 194.818 68.072) (width 1) (layer B.Cu) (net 4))
 (segment (start 204.47 66.802) (end 203.2 68.072) (width 1) (layer B.Cu) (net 4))
 (segment (start 200.66 60.96) (end 200.66 63.5) (width 0.4) (layer B.Cu) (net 12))
 (segment (start 200.66 50.8) (end 201.93 50.8) (width 1) (layer B.Cu) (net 6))
 (segment (start 201.93 50.8) (end 204.47 48.26) (width 1) (layer B.Cu) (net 6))
 (segment (start 204.47 40.64) (end 204.47 48.26) (width 1) (layer B.Cu) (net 6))
 (segment (start 202.946 35.56) (end 202.946 39.116) (width 1) (layer B.Cu) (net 6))
 (segment (start 202.946 39.116) (end 204.47 40.64) (width 1) (layer B.Cu) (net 6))
 (segment (start 224.79 59.69) (end 224.79 63.5) (width 0.4) (layer B.Cu) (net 9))
 (segment (start 219.71 40.64) (end 220.98 40.64) (width 0.4) (layer B.Cu) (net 8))
 (segment (start 226.06 48.26) (end 224.79 49.53) (width 0.4) (layer B.Cu) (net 8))
 (segment (start 226.06 44.45) (end 226.06 48.26) (width 0.4) (layer B.Cu) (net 8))
 (segment (start 224.79 43.18) (end 226.06 44.45) (width 0.4) (layer B.Cu) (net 8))
 (segment (start 223.52 43.18) (end 224.79 43.18) (width 0.4) (layer B.Cu) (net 8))
 (segment (start 220.98 40.64) (end 223.52 43.18) (width 0.4) (layer B.Cu) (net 8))
 (segment (start 221.47784 30.51556) (end 221.47784 39.86784) (width 0.4) (layer B.Cu) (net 8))
 (segment (start 220.70568 40.64) (end 219.71 40.64) (width 0.4) (layer B.Cu) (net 8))
 (segment (start 221.47784 39.86784) (end 220.70568 40.64) (width 0.4) (layer B.Cu) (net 8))
 (segment (start 154.305 30.48) (end 154.305 29.845) (width 1) (layer B.Cu) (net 1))
 (segment (start 173.355 30.48) (end 173.355 29.845) (width 1) (layer B.Cu) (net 1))
 (segment (start 190.5 29.845) (end 203.9874 29.845) (width 1) (layer B.Cu) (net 1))
 (segment (start 203.9874 29.845) (end 204.6478 30.5054) (width 1) (layer B.Cu) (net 1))
 (segment (start 173.355 29.845) (end 190.5 29.845) (width 1) (layer B.Cu) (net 1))
 (segment (start 154.305 29.845) (end 173.355 29.845) (width 1) (layer B.Cu) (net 1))
 (segment (start 143.51 29.845) (end 154.305 29.845) (width 1) (layer B.Cu) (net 1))
 (segment (start 226.58324 35.56762) (end 226.58324 27.19324) (width 1) (layer B.Cu) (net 1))
 (segment (start 226.58324 27.19324) (end 225.425 26.035) (width 1) (layer B.Cu) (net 1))
 (segment (start 225.425 26.035) (end 206.375 26.035) (width 1) (layer B.Cu) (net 1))
 (segment (start 206.375 26.035) (end 204.6478 27.7622) (width 1) (layer B.Cu) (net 1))
 (segment (start 204.6478 27.7622) (end 204.6478 30.5054) (width 1) (layer B.Cu) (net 1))
 (segment (start 163.83 36.83) (end 163.83 33.02) (width 1) (layer B.Cu) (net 2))
 (segment (start 182.88 36.83) (end 182.88 33.02) (width 1) (layer B.Cu) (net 2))
 (segment (start 199.39 33.02) (end 182.88 33.02) (width 1) (layer B.Cu) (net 2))
 (segment (start 182.88 33.02) (end 163.83 33.02) (width 1) (layer B.Cu) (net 2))
 (segment (start 163.83 33.02) (end 145.415 33.02) (width 1) (layer B.Cu) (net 2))
 (segment (start 208.0514 30.5054) (end 208.0514 31.9786) (width 1) (layer B.Cu) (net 2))
 (segment (start 207.01 33.02) (end 199.39 33.02) (width 1) (layer B.Cu) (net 2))
 (segment (start 208.0514 31.9786) (end 207.01 33.02) (width 1) (layer B.Cu) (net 2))
 (segment (start 145.415 33.02) (end 143.51 34.925) (width 1) (layer B.Cu) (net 2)))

